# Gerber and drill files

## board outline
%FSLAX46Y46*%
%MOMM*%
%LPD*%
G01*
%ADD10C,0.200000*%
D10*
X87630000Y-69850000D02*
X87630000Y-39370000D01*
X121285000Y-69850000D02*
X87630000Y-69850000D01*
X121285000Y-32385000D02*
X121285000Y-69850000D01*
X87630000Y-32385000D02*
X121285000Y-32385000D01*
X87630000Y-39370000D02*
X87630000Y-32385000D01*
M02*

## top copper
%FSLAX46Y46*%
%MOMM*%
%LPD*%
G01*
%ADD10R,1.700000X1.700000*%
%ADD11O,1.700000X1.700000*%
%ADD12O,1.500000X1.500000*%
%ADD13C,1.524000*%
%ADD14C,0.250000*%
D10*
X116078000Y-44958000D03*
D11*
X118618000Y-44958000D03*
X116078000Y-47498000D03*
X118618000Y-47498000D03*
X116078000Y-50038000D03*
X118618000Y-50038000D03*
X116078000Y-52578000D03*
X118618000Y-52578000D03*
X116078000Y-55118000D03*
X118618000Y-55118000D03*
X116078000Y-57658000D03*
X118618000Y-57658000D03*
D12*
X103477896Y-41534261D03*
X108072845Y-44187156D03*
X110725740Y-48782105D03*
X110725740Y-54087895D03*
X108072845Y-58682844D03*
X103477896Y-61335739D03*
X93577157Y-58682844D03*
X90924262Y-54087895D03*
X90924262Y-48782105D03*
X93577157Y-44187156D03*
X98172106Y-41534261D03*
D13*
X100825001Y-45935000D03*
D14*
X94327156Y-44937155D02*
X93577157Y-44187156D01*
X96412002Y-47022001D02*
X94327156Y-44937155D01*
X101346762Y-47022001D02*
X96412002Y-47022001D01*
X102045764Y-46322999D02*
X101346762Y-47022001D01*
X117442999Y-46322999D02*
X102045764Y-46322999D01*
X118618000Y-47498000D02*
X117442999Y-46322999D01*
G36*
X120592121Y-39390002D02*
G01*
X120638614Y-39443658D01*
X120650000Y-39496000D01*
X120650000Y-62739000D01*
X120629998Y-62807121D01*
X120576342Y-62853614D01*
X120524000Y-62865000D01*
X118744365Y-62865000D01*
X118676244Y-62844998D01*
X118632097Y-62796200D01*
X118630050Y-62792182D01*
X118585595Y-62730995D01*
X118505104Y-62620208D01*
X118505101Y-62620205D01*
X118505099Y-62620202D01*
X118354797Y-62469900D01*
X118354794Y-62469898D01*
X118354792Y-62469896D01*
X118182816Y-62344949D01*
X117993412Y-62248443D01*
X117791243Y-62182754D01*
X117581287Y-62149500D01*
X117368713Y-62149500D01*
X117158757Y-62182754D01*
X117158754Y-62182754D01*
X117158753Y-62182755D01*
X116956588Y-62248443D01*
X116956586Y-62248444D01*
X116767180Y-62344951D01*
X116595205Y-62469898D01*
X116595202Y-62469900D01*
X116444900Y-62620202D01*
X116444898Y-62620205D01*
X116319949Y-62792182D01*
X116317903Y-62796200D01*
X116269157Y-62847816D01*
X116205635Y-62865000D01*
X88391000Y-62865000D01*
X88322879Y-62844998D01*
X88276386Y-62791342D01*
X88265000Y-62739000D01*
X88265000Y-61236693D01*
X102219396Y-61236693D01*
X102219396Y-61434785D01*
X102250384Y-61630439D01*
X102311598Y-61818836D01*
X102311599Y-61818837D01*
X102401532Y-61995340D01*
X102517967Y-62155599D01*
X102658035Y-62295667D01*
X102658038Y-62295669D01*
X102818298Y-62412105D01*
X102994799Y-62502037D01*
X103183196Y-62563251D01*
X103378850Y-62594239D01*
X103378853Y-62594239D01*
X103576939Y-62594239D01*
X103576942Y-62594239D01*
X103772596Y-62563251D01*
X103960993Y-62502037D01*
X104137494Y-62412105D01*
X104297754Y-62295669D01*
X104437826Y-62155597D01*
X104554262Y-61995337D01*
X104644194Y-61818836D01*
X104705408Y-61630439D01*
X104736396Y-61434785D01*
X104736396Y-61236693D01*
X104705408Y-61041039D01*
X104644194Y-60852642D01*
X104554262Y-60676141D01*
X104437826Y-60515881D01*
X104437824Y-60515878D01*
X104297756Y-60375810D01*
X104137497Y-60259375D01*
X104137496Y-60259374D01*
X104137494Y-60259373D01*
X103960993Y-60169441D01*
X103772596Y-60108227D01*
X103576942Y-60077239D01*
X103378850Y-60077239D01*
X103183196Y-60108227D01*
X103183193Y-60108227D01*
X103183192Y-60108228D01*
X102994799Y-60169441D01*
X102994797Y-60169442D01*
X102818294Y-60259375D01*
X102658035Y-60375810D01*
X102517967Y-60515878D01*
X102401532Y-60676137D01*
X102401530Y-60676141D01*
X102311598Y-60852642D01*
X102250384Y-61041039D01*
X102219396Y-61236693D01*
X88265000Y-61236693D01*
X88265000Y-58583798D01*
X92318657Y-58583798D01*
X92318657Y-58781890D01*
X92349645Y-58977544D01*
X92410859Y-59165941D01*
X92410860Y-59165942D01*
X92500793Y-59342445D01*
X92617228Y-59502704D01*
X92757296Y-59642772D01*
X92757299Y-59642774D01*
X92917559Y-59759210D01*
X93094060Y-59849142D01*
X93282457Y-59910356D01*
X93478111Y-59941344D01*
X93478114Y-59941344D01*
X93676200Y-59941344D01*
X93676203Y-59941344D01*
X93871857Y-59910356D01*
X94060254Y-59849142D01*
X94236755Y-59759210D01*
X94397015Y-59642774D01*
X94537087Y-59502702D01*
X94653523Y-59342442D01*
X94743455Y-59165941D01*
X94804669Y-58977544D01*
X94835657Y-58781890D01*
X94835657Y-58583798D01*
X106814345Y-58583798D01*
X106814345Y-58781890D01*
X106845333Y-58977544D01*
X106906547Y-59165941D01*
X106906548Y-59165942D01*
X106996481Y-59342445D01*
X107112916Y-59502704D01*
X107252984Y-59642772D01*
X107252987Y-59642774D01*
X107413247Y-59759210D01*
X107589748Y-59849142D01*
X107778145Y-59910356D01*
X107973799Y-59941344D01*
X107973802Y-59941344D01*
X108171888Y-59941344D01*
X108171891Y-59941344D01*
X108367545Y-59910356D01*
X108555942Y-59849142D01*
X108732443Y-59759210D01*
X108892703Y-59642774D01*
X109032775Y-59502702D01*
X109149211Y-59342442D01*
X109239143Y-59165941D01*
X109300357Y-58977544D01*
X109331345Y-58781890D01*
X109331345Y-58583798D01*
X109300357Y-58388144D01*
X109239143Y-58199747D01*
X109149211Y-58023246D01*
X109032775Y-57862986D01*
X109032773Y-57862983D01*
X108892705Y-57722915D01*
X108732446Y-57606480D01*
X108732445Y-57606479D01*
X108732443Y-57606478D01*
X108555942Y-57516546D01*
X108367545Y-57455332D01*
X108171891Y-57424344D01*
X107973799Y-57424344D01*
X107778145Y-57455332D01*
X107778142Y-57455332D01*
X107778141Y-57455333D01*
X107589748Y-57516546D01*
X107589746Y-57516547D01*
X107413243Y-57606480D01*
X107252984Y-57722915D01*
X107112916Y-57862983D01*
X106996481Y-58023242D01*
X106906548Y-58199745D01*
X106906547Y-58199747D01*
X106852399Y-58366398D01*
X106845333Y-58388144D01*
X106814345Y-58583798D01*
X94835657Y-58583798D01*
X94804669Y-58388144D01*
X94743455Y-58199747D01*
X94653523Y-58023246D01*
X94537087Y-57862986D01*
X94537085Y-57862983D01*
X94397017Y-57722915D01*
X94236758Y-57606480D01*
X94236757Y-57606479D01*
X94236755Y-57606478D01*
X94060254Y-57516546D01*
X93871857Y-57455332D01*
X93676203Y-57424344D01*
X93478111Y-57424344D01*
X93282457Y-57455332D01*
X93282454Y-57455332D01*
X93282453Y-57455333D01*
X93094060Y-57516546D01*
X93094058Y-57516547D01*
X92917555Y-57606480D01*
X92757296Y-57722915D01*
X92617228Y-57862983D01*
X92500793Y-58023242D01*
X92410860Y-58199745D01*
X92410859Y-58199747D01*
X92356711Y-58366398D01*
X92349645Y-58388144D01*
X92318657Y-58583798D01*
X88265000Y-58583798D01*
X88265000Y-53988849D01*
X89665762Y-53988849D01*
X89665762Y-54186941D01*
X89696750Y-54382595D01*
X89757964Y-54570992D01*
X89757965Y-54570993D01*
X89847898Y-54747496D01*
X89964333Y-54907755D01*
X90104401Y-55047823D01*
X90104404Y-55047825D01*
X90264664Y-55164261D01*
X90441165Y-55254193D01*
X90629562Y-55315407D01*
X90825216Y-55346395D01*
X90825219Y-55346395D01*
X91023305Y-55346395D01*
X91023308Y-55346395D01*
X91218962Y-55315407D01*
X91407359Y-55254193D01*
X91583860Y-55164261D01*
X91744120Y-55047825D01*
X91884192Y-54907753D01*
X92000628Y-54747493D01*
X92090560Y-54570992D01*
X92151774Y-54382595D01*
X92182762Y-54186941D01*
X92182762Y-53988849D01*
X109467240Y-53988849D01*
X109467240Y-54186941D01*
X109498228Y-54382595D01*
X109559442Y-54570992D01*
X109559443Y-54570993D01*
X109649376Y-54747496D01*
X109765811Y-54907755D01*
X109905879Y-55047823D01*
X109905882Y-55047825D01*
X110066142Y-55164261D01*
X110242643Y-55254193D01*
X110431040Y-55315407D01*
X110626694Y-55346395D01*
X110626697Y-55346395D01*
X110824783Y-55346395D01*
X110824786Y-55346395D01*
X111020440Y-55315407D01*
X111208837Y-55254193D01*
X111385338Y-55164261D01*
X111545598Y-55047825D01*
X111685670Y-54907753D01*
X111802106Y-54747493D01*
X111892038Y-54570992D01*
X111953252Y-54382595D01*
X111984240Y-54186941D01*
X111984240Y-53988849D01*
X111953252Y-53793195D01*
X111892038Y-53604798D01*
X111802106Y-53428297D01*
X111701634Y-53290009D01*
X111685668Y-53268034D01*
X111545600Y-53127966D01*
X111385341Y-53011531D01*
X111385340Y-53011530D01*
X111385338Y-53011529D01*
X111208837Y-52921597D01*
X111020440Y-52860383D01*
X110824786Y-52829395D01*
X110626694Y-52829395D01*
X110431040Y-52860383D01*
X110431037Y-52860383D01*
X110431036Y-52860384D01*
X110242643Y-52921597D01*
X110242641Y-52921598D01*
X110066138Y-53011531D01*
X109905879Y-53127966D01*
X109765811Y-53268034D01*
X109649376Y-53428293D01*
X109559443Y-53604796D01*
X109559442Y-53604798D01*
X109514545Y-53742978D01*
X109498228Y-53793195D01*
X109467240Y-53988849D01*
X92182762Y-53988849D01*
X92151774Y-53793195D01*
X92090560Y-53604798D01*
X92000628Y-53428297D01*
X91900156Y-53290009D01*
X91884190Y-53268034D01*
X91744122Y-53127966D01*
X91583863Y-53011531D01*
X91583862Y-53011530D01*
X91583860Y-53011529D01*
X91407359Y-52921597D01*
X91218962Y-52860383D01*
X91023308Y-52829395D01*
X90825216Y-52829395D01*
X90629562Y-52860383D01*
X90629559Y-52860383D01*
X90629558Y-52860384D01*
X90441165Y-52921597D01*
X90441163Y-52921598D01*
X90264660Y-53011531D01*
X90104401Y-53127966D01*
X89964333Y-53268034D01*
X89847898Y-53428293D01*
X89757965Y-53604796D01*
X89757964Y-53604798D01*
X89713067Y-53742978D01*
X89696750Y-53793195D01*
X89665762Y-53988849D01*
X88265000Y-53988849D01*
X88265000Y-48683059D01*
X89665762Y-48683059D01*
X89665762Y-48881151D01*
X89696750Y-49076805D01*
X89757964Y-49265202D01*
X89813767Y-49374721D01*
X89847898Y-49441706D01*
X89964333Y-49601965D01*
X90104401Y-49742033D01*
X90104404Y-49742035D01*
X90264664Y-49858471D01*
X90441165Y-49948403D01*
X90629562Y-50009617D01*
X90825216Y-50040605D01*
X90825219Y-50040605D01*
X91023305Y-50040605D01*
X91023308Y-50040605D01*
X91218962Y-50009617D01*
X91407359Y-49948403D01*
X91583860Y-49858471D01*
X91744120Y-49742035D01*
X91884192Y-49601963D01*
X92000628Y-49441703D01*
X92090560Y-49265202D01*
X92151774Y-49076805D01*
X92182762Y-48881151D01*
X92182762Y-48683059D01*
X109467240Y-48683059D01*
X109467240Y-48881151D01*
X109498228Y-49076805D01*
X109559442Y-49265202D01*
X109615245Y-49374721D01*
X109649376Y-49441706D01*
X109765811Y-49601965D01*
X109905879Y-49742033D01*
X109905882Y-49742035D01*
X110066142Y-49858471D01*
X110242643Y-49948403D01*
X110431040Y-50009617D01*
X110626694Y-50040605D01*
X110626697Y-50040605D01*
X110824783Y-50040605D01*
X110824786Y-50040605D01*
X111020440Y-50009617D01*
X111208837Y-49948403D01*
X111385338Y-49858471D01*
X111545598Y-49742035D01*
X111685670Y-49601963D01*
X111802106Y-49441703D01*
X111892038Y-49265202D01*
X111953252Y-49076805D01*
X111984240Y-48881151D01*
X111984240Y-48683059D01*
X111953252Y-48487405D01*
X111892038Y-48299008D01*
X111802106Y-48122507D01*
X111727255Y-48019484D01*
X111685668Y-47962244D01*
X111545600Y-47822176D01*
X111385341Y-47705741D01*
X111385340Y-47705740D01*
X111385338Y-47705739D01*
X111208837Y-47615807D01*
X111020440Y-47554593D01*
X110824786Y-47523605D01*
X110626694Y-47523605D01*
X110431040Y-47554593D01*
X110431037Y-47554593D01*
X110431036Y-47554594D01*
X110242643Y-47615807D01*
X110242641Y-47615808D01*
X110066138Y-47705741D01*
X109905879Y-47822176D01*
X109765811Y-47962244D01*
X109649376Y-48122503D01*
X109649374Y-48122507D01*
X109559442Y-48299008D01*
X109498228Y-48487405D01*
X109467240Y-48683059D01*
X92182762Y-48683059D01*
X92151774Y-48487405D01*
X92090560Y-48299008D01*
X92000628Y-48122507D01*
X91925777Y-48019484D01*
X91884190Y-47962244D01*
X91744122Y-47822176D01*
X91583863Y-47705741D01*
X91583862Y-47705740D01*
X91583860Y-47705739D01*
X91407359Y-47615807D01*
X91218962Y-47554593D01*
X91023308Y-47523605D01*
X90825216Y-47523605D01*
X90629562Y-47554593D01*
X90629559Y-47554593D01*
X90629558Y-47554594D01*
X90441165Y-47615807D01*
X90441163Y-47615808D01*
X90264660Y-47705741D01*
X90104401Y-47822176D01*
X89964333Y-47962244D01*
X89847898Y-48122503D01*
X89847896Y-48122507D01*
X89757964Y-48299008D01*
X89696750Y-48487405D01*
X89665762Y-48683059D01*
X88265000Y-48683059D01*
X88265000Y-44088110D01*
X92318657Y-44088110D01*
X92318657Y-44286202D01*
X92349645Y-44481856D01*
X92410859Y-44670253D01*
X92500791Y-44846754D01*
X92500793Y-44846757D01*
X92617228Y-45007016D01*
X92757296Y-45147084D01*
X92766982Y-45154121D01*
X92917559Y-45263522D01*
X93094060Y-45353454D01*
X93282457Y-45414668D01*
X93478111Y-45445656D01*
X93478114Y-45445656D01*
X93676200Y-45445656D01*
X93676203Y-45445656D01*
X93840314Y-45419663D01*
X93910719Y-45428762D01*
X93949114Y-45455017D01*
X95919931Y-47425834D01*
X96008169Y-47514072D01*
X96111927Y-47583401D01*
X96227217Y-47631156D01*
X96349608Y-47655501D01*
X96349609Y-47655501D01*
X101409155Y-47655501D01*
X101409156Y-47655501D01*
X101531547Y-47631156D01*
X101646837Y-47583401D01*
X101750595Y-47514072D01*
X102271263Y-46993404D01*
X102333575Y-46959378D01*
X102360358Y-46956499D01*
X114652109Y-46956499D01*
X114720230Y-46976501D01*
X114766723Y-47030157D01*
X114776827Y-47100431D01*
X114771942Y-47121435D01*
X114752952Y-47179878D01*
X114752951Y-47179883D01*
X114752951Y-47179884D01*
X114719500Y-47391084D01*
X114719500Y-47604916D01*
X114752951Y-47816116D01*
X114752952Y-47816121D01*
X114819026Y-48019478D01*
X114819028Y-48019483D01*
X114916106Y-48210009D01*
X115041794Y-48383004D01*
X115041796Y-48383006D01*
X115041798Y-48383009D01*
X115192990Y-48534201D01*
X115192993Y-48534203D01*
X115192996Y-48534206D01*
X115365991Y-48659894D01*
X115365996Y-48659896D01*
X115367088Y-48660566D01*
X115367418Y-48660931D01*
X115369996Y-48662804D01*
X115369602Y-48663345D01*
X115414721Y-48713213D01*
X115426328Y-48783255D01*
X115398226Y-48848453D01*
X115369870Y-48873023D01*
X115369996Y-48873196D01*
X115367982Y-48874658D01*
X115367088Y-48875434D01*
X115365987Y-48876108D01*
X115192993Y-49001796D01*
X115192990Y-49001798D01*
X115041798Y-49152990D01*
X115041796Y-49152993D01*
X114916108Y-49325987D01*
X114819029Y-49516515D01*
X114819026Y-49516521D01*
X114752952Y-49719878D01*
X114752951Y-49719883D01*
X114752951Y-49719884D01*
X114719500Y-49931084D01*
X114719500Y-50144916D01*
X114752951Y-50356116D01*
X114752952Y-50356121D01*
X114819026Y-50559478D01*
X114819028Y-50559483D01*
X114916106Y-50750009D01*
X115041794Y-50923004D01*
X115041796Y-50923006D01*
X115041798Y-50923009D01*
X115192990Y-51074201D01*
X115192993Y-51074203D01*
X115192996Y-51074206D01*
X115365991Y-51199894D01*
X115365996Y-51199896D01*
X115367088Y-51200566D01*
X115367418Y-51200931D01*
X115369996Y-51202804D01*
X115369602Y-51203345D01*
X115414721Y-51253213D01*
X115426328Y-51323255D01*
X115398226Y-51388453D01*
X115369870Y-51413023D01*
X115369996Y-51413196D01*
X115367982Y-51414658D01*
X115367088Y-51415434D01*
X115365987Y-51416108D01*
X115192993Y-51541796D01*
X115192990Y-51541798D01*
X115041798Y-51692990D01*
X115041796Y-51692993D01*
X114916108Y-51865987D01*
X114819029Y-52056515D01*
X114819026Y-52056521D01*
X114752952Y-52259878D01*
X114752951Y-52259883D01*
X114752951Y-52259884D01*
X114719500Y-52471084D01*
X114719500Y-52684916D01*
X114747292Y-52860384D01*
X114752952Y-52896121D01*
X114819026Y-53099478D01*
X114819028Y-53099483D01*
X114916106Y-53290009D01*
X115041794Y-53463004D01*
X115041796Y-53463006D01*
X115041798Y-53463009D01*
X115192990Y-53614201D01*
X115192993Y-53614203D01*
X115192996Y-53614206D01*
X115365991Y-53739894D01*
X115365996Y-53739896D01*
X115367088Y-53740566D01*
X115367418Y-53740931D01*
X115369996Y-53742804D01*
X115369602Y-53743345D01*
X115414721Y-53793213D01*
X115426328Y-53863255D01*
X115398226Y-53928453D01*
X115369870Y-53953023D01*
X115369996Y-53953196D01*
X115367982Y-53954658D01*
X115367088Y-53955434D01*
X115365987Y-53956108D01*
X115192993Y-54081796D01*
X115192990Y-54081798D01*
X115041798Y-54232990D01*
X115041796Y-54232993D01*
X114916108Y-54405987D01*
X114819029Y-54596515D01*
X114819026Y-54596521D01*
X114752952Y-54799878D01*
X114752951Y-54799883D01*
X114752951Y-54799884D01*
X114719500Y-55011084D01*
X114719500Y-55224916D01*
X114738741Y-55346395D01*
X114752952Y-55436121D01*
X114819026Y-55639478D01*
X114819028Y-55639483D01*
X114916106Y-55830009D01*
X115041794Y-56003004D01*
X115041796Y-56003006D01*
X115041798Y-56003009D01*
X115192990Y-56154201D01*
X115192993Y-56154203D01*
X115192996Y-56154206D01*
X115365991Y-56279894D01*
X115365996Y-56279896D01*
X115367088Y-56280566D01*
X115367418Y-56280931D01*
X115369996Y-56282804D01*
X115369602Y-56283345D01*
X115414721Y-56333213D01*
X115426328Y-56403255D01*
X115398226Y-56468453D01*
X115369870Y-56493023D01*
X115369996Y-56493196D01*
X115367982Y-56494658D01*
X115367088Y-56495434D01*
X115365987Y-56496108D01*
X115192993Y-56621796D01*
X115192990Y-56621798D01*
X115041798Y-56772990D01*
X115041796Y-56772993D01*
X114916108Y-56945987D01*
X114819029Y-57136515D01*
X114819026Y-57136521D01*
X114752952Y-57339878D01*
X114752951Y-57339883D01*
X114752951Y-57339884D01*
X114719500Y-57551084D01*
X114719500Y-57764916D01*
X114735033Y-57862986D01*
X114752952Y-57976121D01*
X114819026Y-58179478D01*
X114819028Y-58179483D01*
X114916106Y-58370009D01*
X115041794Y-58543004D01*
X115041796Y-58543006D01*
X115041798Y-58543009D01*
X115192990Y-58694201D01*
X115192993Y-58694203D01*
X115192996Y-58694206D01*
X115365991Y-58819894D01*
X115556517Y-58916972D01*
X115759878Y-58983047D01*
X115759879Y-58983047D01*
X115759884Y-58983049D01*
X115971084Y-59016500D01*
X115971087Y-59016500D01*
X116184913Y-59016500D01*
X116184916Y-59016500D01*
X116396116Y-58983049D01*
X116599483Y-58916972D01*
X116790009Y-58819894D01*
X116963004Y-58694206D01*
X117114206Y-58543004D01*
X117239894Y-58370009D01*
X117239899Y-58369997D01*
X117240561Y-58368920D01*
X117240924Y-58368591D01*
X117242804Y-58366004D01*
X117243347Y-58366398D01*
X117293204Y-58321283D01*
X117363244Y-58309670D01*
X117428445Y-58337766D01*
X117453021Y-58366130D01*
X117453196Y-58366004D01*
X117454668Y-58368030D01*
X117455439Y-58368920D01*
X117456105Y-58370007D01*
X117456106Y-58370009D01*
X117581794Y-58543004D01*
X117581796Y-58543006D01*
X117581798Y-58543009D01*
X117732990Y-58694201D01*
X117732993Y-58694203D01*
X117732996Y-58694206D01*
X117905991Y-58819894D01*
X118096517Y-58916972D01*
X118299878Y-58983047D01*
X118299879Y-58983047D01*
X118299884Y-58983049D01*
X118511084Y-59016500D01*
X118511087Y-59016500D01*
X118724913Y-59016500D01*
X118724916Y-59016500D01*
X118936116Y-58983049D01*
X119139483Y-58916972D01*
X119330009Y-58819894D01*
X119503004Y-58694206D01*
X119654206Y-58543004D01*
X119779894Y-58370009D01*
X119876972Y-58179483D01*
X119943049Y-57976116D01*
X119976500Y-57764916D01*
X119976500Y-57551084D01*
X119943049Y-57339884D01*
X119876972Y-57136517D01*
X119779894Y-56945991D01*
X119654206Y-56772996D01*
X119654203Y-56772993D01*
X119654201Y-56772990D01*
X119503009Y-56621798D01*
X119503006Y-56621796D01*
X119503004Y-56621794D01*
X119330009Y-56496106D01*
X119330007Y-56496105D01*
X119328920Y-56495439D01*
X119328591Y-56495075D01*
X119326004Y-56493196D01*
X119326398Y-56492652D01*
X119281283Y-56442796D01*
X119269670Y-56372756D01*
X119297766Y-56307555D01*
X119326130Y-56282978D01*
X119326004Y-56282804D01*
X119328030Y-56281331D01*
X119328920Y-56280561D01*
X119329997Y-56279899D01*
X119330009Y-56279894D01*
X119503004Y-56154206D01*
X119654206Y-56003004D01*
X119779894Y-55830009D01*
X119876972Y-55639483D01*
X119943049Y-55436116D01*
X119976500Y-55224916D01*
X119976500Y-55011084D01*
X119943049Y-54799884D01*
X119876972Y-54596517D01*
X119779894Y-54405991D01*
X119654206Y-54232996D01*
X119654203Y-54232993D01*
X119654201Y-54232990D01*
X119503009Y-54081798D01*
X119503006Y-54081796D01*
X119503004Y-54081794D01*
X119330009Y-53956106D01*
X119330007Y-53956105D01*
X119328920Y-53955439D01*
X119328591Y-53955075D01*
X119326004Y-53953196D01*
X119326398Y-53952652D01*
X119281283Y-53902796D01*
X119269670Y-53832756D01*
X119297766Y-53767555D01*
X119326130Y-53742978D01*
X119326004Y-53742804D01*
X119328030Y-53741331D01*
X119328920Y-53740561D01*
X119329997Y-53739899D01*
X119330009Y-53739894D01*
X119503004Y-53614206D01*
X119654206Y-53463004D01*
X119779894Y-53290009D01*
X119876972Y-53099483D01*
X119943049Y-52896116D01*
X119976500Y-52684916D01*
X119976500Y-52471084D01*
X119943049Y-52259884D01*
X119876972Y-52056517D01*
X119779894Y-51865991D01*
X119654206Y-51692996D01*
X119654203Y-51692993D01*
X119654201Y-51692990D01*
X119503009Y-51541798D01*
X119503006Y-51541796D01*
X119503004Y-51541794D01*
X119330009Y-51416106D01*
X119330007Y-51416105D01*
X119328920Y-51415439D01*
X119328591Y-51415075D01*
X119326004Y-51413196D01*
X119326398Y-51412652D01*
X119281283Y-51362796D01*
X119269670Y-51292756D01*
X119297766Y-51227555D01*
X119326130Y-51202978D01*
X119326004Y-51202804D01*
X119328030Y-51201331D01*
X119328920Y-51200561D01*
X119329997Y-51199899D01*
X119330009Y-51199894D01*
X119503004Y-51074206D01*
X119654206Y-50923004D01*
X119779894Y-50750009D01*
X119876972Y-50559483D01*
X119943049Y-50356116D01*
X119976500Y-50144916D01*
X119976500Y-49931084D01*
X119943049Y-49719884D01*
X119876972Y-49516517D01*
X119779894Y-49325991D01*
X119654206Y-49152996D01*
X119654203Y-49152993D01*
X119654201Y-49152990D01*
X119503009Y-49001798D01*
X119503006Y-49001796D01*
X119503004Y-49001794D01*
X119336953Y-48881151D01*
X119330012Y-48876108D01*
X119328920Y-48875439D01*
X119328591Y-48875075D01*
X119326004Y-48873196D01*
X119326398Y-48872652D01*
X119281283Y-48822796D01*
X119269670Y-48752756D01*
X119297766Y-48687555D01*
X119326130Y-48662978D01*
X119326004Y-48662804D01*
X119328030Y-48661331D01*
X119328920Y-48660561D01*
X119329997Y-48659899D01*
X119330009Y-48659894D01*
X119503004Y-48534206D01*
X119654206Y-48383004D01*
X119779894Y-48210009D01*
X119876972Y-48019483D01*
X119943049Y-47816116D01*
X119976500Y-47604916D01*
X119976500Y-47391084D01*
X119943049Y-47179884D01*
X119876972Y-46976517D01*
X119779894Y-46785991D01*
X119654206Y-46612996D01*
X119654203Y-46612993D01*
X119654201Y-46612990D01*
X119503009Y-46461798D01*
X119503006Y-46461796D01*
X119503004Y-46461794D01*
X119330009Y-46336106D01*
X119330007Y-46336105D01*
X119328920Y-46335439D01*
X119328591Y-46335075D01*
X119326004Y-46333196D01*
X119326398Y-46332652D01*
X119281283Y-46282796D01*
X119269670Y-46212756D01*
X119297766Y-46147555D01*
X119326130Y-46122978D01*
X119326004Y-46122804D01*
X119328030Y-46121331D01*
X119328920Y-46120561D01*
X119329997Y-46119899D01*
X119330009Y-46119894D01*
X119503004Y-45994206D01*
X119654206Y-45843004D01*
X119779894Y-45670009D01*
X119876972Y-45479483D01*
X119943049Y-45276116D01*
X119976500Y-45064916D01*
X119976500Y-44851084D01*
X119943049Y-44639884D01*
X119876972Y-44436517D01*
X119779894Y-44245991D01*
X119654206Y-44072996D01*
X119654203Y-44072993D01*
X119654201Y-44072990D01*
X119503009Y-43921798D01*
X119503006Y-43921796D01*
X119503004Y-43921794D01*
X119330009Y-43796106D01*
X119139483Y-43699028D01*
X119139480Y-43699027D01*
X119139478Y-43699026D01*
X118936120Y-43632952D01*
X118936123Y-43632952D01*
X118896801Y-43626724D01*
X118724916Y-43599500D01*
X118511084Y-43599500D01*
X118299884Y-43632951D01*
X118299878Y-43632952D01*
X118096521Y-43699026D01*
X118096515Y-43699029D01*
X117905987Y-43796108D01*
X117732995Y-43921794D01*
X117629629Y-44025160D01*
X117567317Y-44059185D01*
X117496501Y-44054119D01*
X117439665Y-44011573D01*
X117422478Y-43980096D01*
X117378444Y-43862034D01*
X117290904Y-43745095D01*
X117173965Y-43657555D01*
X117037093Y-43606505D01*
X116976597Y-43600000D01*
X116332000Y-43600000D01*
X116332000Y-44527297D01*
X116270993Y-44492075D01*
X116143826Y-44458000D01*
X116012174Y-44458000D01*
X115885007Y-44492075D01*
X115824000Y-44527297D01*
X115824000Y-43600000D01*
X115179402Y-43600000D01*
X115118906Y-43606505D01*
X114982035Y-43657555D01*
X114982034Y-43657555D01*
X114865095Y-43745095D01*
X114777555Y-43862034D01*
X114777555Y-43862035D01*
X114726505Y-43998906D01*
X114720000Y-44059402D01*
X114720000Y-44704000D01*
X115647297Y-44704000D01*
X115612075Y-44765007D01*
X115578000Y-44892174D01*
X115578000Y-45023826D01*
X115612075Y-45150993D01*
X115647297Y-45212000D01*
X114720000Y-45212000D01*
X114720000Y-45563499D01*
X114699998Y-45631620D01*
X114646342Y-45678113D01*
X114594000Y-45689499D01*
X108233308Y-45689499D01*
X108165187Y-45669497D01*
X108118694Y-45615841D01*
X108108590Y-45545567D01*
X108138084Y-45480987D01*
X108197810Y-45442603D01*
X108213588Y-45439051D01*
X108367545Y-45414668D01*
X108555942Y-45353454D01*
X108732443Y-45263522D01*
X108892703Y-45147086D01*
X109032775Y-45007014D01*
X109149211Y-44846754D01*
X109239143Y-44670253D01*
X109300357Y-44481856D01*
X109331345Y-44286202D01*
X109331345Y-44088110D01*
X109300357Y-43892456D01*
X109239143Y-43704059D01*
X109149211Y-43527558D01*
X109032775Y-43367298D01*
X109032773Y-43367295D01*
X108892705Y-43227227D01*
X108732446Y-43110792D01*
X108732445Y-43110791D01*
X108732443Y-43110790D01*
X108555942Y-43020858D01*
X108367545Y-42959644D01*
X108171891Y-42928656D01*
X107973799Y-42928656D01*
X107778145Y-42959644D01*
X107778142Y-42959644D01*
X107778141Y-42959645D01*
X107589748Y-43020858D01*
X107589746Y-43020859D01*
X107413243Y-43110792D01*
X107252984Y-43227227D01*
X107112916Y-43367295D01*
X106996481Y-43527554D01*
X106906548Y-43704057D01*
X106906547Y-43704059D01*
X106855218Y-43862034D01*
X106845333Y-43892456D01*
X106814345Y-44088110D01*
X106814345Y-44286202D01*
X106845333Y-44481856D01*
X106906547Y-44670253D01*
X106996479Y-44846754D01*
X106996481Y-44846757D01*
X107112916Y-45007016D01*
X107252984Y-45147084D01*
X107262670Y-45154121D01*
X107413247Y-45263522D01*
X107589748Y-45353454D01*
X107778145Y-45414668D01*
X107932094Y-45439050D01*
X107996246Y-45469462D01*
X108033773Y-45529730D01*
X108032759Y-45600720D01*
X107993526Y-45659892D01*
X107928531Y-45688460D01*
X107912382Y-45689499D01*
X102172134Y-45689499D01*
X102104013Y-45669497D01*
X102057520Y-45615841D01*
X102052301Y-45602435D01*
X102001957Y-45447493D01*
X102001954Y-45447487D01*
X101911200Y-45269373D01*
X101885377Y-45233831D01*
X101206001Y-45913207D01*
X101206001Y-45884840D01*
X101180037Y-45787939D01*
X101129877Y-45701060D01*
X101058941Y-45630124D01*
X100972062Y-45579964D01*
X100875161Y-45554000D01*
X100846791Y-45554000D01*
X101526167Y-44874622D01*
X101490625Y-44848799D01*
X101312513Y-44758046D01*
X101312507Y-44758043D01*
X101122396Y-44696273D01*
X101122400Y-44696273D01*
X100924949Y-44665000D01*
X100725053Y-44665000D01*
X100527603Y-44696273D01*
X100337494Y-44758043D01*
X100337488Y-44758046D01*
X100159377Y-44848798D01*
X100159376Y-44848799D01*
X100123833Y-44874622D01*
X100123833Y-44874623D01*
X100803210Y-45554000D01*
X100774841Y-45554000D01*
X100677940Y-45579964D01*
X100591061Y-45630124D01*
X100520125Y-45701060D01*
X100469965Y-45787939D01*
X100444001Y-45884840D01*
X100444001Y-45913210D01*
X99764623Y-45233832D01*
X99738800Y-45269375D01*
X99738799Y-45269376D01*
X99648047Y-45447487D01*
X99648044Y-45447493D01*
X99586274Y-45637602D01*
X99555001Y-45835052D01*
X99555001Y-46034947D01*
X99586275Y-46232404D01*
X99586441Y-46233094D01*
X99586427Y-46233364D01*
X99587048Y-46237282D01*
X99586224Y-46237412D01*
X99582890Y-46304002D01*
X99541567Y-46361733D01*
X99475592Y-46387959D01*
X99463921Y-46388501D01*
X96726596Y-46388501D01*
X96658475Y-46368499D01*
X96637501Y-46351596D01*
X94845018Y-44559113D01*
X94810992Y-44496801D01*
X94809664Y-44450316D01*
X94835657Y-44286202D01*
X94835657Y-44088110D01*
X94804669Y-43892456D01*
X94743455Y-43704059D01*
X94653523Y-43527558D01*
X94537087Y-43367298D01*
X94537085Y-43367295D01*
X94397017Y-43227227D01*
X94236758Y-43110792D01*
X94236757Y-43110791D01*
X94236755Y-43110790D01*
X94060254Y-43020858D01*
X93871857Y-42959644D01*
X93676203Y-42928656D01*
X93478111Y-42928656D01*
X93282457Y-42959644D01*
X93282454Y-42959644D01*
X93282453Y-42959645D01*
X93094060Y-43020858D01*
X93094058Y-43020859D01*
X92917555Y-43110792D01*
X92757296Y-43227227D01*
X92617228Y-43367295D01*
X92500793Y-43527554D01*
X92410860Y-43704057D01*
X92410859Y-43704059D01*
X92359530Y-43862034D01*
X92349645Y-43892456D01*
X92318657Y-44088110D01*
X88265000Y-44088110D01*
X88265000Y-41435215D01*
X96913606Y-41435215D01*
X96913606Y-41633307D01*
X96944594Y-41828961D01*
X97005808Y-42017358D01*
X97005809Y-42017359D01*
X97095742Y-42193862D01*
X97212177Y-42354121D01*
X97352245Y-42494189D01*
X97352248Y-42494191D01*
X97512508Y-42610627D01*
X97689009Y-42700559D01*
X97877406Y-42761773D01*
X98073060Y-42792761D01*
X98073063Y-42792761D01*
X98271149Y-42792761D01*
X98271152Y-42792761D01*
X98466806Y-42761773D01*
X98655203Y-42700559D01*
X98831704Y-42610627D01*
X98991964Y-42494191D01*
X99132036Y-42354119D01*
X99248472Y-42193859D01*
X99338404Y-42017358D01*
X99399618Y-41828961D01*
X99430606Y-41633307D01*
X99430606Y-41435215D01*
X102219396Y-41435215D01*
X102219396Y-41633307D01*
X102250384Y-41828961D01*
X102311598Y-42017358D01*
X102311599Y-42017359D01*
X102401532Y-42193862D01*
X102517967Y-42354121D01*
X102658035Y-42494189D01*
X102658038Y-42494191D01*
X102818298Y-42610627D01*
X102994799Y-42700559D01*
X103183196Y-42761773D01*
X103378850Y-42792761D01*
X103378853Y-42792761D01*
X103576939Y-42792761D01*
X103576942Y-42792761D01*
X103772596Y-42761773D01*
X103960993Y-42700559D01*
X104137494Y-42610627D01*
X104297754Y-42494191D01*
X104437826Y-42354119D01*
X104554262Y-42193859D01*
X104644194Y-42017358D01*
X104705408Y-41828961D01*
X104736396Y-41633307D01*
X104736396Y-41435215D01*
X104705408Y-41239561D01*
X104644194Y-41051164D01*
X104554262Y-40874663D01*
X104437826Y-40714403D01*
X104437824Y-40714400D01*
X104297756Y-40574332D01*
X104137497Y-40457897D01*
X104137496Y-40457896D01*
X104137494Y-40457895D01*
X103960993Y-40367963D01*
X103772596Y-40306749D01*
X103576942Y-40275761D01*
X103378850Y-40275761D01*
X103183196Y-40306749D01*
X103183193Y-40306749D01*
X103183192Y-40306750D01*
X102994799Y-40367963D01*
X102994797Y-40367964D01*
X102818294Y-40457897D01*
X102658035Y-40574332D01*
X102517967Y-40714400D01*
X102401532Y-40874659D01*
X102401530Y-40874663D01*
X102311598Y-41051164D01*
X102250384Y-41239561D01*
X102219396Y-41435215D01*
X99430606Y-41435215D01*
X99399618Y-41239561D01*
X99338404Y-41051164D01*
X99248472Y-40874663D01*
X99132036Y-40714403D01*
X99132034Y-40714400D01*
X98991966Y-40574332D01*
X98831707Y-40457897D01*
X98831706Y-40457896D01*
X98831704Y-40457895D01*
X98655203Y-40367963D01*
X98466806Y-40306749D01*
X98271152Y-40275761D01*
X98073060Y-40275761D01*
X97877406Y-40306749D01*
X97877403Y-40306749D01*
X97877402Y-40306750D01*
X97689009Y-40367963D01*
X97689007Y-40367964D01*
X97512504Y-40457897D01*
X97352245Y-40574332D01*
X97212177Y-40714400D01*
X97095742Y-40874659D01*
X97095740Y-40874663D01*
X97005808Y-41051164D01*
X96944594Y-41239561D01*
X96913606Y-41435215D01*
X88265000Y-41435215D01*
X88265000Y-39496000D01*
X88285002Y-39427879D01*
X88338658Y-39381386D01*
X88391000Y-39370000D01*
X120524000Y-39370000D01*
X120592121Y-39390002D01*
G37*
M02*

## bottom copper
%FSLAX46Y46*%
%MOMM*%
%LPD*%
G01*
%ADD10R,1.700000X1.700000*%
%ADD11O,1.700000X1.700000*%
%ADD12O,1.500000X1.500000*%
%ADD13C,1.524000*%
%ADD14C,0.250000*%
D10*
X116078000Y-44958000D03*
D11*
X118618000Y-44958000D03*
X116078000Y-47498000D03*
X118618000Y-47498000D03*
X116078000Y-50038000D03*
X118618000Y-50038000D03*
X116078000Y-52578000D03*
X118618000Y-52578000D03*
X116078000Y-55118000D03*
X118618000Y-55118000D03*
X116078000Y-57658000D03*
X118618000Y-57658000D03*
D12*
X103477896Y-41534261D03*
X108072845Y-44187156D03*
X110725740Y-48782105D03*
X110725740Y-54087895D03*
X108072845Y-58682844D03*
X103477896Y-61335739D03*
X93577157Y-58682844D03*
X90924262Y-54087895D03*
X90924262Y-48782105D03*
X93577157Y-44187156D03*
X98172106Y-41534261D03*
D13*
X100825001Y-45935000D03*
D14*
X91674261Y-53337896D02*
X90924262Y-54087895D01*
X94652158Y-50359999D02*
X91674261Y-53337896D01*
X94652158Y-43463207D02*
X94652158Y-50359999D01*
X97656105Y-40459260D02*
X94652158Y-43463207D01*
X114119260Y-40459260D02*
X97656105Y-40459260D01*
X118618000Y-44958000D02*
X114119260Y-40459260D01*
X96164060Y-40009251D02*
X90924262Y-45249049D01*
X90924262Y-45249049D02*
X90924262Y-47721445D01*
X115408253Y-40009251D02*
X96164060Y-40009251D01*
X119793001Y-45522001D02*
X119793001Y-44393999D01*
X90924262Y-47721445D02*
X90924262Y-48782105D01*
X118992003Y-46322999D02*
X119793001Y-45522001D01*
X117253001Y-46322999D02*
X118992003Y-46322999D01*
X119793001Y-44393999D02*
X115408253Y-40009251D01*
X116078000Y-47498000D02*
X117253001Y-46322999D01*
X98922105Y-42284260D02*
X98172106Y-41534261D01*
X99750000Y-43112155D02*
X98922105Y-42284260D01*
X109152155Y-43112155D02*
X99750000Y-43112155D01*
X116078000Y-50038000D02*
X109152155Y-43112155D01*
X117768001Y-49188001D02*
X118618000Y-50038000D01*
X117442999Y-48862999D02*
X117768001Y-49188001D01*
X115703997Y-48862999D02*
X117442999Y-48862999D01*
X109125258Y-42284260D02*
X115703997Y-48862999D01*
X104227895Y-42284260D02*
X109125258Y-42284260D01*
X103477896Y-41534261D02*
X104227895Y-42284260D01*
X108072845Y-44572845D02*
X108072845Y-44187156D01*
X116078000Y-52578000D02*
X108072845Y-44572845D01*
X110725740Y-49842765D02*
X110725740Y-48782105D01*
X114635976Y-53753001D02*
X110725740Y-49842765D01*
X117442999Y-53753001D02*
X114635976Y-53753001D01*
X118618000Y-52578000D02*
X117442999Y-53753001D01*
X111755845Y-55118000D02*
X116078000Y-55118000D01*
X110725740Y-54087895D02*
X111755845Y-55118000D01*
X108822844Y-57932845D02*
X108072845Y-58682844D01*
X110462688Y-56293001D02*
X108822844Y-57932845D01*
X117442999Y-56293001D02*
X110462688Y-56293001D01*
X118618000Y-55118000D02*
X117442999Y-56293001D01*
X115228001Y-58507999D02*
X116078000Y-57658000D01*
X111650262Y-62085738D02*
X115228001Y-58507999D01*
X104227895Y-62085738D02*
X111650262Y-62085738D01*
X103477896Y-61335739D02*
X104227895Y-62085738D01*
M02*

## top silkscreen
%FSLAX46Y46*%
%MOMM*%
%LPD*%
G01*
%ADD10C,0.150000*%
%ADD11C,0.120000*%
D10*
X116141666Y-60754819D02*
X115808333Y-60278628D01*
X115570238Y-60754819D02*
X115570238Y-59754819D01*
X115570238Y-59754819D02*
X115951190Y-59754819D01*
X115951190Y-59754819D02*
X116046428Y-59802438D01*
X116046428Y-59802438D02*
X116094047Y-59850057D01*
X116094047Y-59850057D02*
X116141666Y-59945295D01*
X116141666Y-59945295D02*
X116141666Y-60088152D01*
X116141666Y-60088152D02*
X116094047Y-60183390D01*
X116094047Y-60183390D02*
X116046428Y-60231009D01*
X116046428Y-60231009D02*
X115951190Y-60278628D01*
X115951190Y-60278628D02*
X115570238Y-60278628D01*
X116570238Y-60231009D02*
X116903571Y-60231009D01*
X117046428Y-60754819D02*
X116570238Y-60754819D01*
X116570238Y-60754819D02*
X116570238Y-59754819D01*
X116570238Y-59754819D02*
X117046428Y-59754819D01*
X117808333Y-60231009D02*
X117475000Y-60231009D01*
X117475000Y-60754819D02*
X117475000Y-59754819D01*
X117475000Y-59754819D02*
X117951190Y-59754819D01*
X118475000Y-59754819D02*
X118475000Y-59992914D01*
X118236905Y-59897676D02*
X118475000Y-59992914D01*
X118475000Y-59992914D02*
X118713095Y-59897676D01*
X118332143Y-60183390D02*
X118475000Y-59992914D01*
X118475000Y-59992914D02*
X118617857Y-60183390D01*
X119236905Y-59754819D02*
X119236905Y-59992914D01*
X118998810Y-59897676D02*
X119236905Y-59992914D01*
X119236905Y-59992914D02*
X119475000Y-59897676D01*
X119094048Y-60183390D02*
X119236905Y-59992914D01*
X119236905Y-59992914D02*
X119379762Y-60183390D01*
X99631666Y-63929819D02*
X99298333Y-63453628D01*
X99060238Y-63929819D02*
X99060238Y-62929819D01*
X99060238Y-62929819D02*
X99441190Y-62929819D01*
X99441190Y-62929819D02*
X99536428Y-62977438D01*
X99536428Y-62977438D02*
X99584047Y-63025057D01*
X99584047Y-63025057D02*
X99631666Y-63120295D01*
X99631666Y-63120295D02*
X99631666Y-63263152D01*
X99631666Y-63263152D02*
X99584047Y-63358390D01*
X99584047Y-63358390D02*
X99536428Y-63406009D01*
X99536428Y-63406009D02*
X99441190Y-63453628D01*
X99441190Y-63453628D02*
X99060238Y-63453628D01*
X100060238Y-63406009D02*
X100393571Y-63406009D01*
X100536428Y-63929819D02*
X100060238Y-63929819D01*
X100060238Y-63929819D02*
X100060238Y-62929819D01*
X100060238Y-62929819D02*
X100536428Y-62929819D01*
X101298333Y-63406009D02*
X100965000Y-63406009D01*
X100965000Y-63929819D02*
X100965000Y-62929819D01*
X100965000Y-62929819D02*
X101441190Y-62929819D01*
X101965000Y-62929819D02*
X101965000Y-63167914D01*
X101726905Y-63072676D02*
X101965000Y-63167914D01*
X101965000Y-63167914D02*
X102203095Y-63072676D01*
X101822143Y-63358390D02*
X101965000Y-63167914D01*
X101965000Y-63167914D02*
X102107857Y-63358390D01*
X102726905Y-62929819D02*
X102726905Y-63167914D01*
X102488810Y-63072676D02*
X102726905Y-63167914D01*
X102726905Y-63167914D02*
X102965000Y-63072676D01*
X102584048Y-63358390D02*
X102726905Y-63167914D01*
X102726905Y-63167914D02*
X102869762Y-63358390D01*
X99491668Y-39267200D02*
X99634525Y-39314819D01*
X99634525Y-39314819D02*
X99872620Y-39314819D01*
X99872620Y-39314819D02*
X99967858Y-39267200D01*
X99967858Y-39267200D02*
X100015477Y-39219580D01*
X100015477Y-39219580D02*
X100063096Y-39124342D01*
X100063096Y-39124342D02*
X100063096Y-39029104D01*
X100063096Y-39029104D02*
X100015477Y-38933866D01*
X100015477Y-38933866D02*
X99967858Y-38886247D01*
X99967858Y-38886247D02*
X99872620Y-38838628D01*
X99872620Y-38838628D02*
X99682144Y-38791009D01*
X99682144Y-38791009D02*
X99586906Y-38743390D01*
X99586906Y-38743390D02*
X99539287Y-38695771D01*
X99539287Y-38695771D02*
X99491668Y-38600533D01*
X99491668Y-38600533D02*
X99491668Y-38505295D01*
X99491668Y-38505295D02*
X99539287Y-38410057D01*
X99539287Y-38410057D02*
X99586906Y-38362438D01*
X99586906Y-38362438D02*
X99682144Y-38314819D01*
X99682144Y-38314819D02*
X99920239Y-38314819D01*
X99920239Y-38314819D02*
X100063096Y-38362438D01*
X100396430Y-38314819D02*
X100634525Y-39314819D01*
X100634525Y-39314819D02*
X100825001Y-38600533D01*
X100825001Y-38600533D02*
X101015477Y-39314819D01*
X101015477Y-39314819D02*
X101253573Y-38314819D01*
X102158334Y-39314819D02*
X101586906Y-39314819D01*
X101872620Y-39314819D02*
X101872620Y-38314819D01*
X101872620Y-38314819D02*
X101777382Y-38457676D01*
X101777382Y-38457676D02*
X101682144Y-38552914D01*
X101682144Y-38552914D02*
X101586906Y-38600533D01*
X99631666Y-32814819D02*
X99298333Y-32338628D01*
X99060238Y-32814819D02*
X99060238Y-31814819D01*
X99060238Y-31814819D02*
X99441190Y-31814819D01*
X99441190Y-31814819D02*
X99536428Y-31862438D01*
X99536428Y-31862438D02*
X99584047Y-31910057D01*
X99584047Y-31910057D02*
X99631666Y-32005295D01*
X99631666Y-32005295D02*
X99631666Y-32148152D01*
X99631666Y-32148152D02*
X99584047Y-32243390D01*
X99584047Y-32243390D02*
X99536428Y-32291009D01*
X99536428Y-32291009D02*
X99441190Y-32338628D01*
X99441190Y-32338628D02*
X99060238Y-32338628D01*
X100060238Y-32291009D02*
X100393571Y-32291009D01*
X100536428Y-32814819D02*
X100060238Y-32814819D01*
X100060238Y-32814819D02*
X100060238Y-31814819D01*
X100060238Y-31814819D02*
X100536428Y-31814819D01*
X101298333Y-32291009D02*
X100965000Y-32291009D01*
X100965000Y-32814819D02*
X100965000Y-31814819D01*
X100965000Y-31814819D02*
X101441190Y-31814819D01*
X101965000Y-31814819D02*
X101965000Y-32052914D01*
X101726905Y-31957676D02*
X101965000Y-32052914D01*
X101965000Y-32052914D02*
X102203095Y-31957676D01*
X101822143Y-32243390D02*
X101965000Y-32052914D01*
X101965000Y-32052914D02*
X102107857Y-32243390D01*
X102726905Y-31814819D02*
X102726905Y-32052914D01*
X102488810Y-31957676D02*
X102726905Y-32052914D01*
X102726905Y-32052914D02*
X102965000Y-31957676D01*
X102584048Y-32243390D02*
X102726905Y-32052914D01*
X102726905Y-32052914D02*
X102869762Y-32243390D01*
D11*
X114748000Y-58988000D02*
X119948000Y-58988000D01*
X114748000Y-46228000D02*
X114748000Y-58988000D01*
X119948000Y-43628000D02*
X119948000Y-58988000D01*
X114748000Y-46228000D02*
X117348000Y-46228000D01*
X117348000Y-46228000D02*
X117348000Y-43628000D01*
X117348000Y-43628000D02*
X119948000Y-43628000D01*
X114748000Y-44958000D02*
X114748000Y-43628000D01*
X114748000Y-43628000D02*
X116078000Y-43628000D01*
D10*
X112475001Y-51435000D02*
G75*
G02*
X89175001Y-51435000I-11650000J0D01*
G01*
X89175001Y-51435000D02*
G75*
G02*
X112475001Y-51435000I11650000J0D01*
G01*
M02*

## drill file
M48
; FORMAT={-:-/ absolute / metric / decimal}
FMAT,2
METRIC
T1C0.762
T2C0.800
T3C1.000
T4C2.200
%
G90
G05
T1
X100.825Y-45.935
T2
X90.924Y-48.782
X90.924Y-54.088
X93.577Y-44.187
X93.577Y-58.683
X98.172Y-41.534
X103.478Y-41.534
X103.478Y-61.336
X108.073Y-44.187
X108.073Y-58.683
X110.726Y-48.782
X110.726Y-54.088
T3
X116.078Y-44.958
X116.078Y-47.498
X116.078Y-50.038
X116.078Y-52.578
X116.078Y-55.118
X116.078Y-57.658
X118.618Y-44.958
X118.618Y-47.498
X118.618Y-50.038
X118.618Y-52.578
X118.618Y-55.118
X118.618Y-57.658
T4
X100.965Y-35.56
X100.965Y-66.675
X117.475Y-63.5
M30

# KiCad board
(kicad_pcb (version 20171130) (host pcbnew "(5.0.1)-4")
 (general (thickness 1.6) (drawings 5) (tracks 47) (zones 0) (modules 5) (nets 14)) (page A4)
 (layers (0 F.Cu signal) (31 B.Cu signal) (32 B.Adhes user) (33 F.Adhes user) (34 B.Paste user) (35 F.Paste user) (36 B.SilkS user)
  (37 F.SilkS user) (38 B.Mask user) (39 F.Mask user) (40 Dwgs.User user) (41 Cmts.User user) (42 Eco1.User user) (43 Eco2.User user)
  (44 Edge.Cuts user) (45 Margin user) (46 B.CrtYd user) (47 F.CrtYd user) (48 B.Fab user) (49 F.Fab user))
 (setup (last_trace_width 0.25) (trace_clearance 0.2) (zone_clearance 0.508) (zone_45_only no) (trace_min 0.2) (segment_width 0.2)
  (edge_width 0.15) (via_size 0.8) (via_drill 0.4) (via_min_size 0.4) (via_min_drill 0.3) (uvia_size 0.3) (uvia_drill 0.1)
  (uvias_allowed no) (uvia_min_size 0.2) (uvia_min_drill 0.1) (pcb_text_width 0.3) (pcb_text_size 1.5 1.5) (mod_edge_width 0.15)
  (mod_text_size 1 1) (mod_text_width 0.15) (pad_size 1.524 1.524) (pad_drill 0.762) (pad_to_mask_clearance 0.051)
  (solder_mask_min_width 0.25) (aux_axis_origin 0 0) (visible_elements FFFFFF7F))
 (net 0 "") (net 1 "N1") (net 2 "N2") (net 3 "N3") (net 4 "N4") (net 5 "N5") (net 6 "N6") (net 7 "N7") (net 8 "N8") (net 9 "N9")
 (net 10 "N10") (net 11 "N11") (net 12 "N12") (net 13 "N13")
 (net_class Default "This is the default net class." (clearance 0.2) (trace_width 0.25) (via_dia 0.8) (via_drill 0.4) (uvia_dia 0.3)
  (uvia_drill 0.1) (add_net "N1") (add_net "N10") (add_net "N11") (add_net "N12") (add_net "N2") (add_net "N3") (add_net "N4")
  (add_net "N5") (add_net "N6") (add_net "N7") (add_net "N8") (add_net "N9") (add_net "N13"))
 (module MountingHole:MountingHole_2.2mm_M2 (layer F.Cu) (at 117.475 63.5)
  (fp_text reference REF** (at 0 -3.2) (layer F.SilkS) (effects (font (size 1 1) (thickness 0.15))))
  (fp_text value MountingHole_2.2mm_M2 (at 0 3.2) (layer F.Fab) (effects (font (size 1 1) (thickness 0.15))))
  (pad 1 np_thru_hole circle (at 0 0) (size 2.2 2.2) (drill 2.2) (layers *.Cu *.Mask)))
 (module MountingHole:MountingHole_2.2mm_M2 (layer F.Cu) (at 100.965 66.675)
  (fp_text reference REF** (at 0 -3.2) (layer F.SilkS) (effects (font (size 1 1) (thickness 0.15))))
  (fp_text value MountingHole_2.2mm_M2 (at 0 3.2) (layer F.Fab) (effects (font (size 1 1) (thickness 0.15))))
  (pad 1 np_thru_hole circle (at 0 0) (size 2.2 2.2) (drill 2.2) (layers *.Cu *.Mask)))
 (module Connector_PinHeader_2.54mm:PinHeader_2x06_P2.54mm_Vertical (layer F.Cu) (at 116.078 44.958)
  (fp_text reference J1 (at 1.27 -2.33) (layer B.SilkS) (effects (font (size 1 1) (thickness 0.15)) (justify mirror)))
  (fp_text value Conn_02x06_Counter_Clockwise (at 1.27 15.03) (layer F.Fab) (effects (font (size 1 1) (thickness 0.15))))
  (fp_line (start -1.33 14.03) (end 3.87 14.03) (layer F.SilkS) (width 0.12))
  (fp_line (start -1.33 1.27) (end -1.33 14.03) (layer F.SilkS) (width 0.12))
  (fp_line (start 3.87 -1.33) (end 3.87 14.03) (layer F.SilkS) (width 0.12))
  (fp_line (start -1.33 1.27) (end 1.27 1.27) (layer F.SilkS) (width 0.12))
  (fp_line (start 1.27 1.27) (end 1.27 -1.33) (layer F.SilkS) (width 0.12))
  (fp_line (start 1.27 -1.33) (end 3.87 -1.33) (layer F.SilkS) (width 0.12))
  (fp_line (start -1.33 0) (end -1.33 -1.33) (layer F.SilkS) (width 0.12))
  (fp_line (start -1.33 -1.33) (end 0 -1.33) (layer F.SilkS) (width 0.12))
  (pad 1 thru_hole rect (at 0 0) (size 1.7 1.7) (drill 1) (layers *.Cu *.Mask) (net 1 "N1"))
  (pad 2 thru_hole oval (at 2.54 0) (size 1.7 1.7) (drill 1) (layers *.Cu *.Mask) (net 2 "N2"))
  (pad 3 thru_hole oval (at 0 2.54) (size 1.7 1.7) (drill 1) (layers *.Cu *.Mask) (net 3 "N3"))
  (pad 4 thru_hole oval (at 2.54 2.54) (size 1.7 1.7) (drill 1) (layers *.Cu *.Mask) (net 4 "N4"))
  (pad 5 thru_hole oval (at 0 5.08) (size 1.7 1.7) (drill 1) (layers *.Cu *.Mask) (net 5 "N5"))
  (pad 6 thru_hole oval (at 2.54 5.08) (size 1.7 1.7) (drill 1) (layers *.Cu *.Mask) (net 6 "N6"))
  (pad 7 thru_hole oval (at 0 7.62) (size 1.7 1.7) (drill 1) (layers *.Cu *.Mask) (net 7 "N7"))
  (pad 8 thru_hole oval (at 2.54 7.62) (size 1.7 1.7) (drill 1) (layers *.Cu *.Mask) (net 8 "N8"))
  (pad 9 thru_hole oval (at 0 10.16) (size 1.7 1.7) (drill 1) (layers *.Cu *.Mask) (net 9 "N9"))
  (pad 10 thru_hole oval (at 2.54 10.16) (size 1.7 1.7) (drill 1) (layers *.Cu *.Mask) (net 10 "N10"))
  (pad 11 thru_hole oval (at 0 12.7) (size 1.7 1.7) (drill 1) (layers *.Cu *.Mask) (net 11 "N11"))
  (pad 12 thru_hole oval (at 2.54 12.7) (size 1.7 1.7) (drill 1) (layers *.Cu *.Mask) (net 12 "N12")))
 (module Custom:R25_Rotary (layer F.Cu) (at 100.825001 51.435)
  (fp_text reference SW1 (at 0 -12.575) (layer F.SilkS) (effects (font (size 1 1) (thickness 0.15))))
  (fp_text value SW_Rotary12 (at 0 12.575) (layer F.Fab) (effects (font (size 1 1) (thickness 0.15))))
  (fp_circle (center 0 0) (end 0 11.65) (layer F.SilkS) (width 0.15))
  (pad 6 thru_hole oval (at 2.652895 -9.900739) (size 1.5 1.5) (drill 0.8) (layers *.Cu *.Mask) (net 6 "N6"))
  (pad 7 thru_hole oval (at 7.247844 -7.247844) (size 1.5 1.5) (drill 0.8) (layers *.Cu *.Mask) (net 7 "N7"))
  (pad 8 thru_hole oval (at 9.900739 -2.652895) (size 1.5 1.5) (drill 0.8) (layers *.Cu *.Mask) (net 8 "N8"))
  (pad 9 thru_hole oval (at 9.900739 2.652895) (size 1.5 1.5) (drill 0.8) (layers *.Cu *.Mask) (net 9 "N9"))
  (pad 10 thru_hole oval (at 7.247844 7.247844) (size 1.5 1.5) (drill 0.8) (layers *.Cu *.Mask) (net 10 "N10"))
  (pad 11 thru_hole oval (at 2.652895 9.900739) (size 1.5 1.5) (drill 0.8) (layers *.Cu *.Mask) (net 11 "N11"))
  (pad 1 thru_hole oval (at -7.247844 7.247844) (size 1.5 1.5) (drill 0.8) (layers *.Cu *.Mask) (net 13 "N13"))
  (pad 2 thru_hole oval (at -9.900739 2.652895) (size 1.5 1.5) (drill 0.8) (layers *.Cu *.Mask) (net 2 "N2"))
  (pad 3 thru_hole oval (at -9.900739 -2.652895) (size 1.5 1.5) (drill 0.8) (layers *.Cu *.Mask) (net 3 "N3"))
  (pad 4 thru_hole oval (at -7.247844 -7.247844) (size 1.5 1.5) (drill 0.8) (layers *.Cu *.Mask) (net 4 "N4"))
  (pad 5 thru_hole oval (at -2.652895 -9.900739) (size 1.5 1.5) (drill 0.8) (layers *.Cu *.Mask) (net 5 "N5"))
  (pad 13 thru_hole circle (at 0 -5.5) (size 1.524 1.524) (drill 0.762) (layers *.Cu *.Mask) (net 1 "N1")))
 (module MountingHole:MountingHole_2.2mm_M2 (layer F.Cu) (at 100.965 35.56)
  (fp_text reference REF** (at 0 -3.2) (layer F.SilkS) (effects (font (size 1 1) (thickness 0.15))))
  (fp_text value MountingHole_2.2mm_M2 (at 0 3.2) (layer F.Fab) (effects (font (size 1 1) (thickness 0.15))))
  (pad 1 np_thru_hole circle (at 0 0) (size 2.2 2.2) (drill 2.2) (layers *.Cu *.Mask)))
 (gr_line (start 87.63 69.85) (end 87.63 39.37) (layer Edge.Cuts) (width 0.2))
 (gr_line (start 121.285 69.85) (end 87.63 69.85) (layer Edge.Cuts) (width 0.2))
 (gr_line (start 121.285 32.385) (end 121.285 69.85) (layer Edge.Cuts) (width 0.2))
 (gr_line (start 87.63 32.385) (end 121.285 32.385) (layer Edge.Cuts) (width 0.2))
 (gr_line (start 87.63 39.37) (end 87.63 32.385) (layer Edge.Cuts) (width 0.2))
 (segment (start 91.674261 53.337896) (end 90.924262 54.087895) (width 0.25) (layer B.Cu) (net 2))
 (segment (start 94.652158 50.359999) (end 91.674261 53.337896) (width 0.25) (layer B.Cu) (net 2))
 (segment (start 94.652158 43.463207) (end 94.652158 50.359999) (width 0.25) (layer B.Cu) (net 2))
 (segment (start 97.656105 40.45926) (end 94.652158 43.463207) (width 0.25) (layer B.Cu) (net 2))
 (segment (start 114.11926 40.45926) (end 97.656105 40.45926) (width 0.25) (layer B.Cu) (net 2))
 (segment (start 118.618 44.958) (end 114.11926 40.45926) (width 0.25) (layer B.Cu) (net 2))
 (segment (start 96.16406 40.009251) (end 90.924262 45.249049) (width 0.25) (layer B.Cu) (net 3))
 (segment (start 90.924262 45.249049) (end 90.924262 47.721445) (width 0.25) (layer B.Cu) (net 3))
 (segment (start 115.408253 40.009251) (end 96.16406 40.009251) (width 0.25) (layer B.Cu) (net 3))
 (segment (start 119.793001 45.522001) (end 119.793001 44.393999) (width 0.25) (layer B.Cu) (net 3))
 (segment (start 90.924262 47.721445) (end 90.924262 48.782105) (width 0.25) (layer B.Cu) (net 3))
 (segment (start 118.992003 46.322999) (end 119.793001 45.522001) (width 0.25) (layer B.Cu) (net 3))
 (segment (start 117.253001 46.322999) (end 118.992003 46.322999) (width 0.25) (layer B.Cu) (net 3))
 (segment (start 119.793001 44.393999) (end 115.408253 40.009251) (width 0.25) (layer B.Cu) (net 3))
 (segment (start 116.078 47.498) (end 117.253001 46.322999) (width 0.25) (layer B.Cu) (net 3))
 (segment (start 94.327156 44.937155) (end 93.577157 44.187156) (width 0.25) (layer F.Cu) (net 4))
 (segment (start 96.412002 47.022001) (end 94.327156 44.937155) (width 0.25) (layer F.Cu) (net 4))
 (segment (start 101.346762 47.022001) (end 96.412002 47.022001) (width 0.25) (layer F.Cu) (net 4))
 (segment (start 102.045764 46.322999) (end 101.346762 47.022001) (width 0.25) (layer F.Cu) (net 4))
 (segment (start 117.442999 46.322999) (end 102.045764 46.322999) (width 0.25) (layer F.Cu) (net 4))
 (segment (start 118.618 47.498) (end 117.442999 46.322999) (width 0.25) (layer F.Cu) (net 4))
 (segment (start 98.922105 42.28426) (end 98.172106 41.534261) (width 0.25) (layer B.Cu) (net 5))
 (segment (start 99.75 43.112155) (end 98.922105 42.28426) (width 0.25) (layer B.Cu) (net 5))
 (segment (start 109.152155 43.112155) (end 99.75 43.112155) (width 0.25) (layer B.Cu) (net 5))
 (segment (start 116.078 50.038) (end 109.152155 43.112155) (width 0.25) (layer B.Cu) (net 5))
 (segment (start 117.768001 49.188001) (end 118.618 50.038) (width 0.25) (layer B.Cu) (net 6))
 (segment (start 117.442999 48.862999) (end 117.768001 49.188001) (width 0.25) (layer B.Cu) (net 6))
 (segment (start 115.703997 48.862999) (end 117.442999 48.862999) (width 0.25) (layer B.Cu) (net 6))
 (segment (start 109.125258 42.28426) (end 115.703997 48.862999) (width 0.25) (layer B.Cu) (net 6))
 (segment (start 104.227895 42.28426) (end 109.125258 42.28426) (width 0.25) (layer B.Cu) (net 6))
 (segment (start 103.477896 41.534261) (end 104.227895 42.28426) (width 0.25) (layer B.Cu) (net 6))
 (segment (start 108.072845 44.572845) (end 108.072845 44.187156) (width 0.25) (layer B.Cu) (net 7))
 (segment (start 116.078 52.578) (end 108.072845 44.572845) (width 0.25) (layer B.Cu) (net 7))
 (segment (start 110.72574 49.842765) (end 110.72574 48.782105) (width 0.25) (layer B.Cu) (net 8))
 (segment (start 114.635976 53.753001) (end 110.72574 49.842765) (width 0.25) (layer B.Cu) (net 8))
 (segment (start 117.442999 53.753001) (end 114.635976 53.753001) (width 0.25) (layer B.Cu) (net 8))
 (segment (start 118.618 52.578) (end 117.442999 53.753001) (width 0.25) (layer B.Cu) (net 8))
 (segment (start 111.755845 55.118) (end 116.078 55.118) (width 0.25) (layer B.Cu) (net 9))
 (segment (start 110.72574 54.087895) (end 111.755845 55.118) (width 0.25) (layer B.Cu) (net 9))
 (segment (start 108.822844 57.932845) (end 108.072845 58.682844) (width 0.25) (layer B.Cu) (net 10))
 (segment (start 110.462688 56.293001) (end 108.822844 57.932845) (width 0.25) (layer B.Cu) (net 10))
 (segment (start 117.442999 56.293001) (end 110.462688 56.293001) (width 0.25) (layer B.Cu) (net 10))
 (segment (start 118.618 55.118) (end 117.442999 56.293001) (width 0.25) (layer B.Cu) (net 10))
 (segment (start 115.228001 58.507999) (end 116.078 57.658) (width 0.25) (layer B.Cu) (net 11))
 (segment (start 111.650262 62.085738) (end 115.228001 58.507999) (width 0.25) (layer B.Cu) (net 11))
 (segment (start 104.227895 62.085738) (end 111.650262 62.085738) (width 0.25) (layer B.Cu) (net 11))
 (segment (start 103.477896 61.335739) (end 104.227895 62.085738) (width 0.25) (layer B.Cu) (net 11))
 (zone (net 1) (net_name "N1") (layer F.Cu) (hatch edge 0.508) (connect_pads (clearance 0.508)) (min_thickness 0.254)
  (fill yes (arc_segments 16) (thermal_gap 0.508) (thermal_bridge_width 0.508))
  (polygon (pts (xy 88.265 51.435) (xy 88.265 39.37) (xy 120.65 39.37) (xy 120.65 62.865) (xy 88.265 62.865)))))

